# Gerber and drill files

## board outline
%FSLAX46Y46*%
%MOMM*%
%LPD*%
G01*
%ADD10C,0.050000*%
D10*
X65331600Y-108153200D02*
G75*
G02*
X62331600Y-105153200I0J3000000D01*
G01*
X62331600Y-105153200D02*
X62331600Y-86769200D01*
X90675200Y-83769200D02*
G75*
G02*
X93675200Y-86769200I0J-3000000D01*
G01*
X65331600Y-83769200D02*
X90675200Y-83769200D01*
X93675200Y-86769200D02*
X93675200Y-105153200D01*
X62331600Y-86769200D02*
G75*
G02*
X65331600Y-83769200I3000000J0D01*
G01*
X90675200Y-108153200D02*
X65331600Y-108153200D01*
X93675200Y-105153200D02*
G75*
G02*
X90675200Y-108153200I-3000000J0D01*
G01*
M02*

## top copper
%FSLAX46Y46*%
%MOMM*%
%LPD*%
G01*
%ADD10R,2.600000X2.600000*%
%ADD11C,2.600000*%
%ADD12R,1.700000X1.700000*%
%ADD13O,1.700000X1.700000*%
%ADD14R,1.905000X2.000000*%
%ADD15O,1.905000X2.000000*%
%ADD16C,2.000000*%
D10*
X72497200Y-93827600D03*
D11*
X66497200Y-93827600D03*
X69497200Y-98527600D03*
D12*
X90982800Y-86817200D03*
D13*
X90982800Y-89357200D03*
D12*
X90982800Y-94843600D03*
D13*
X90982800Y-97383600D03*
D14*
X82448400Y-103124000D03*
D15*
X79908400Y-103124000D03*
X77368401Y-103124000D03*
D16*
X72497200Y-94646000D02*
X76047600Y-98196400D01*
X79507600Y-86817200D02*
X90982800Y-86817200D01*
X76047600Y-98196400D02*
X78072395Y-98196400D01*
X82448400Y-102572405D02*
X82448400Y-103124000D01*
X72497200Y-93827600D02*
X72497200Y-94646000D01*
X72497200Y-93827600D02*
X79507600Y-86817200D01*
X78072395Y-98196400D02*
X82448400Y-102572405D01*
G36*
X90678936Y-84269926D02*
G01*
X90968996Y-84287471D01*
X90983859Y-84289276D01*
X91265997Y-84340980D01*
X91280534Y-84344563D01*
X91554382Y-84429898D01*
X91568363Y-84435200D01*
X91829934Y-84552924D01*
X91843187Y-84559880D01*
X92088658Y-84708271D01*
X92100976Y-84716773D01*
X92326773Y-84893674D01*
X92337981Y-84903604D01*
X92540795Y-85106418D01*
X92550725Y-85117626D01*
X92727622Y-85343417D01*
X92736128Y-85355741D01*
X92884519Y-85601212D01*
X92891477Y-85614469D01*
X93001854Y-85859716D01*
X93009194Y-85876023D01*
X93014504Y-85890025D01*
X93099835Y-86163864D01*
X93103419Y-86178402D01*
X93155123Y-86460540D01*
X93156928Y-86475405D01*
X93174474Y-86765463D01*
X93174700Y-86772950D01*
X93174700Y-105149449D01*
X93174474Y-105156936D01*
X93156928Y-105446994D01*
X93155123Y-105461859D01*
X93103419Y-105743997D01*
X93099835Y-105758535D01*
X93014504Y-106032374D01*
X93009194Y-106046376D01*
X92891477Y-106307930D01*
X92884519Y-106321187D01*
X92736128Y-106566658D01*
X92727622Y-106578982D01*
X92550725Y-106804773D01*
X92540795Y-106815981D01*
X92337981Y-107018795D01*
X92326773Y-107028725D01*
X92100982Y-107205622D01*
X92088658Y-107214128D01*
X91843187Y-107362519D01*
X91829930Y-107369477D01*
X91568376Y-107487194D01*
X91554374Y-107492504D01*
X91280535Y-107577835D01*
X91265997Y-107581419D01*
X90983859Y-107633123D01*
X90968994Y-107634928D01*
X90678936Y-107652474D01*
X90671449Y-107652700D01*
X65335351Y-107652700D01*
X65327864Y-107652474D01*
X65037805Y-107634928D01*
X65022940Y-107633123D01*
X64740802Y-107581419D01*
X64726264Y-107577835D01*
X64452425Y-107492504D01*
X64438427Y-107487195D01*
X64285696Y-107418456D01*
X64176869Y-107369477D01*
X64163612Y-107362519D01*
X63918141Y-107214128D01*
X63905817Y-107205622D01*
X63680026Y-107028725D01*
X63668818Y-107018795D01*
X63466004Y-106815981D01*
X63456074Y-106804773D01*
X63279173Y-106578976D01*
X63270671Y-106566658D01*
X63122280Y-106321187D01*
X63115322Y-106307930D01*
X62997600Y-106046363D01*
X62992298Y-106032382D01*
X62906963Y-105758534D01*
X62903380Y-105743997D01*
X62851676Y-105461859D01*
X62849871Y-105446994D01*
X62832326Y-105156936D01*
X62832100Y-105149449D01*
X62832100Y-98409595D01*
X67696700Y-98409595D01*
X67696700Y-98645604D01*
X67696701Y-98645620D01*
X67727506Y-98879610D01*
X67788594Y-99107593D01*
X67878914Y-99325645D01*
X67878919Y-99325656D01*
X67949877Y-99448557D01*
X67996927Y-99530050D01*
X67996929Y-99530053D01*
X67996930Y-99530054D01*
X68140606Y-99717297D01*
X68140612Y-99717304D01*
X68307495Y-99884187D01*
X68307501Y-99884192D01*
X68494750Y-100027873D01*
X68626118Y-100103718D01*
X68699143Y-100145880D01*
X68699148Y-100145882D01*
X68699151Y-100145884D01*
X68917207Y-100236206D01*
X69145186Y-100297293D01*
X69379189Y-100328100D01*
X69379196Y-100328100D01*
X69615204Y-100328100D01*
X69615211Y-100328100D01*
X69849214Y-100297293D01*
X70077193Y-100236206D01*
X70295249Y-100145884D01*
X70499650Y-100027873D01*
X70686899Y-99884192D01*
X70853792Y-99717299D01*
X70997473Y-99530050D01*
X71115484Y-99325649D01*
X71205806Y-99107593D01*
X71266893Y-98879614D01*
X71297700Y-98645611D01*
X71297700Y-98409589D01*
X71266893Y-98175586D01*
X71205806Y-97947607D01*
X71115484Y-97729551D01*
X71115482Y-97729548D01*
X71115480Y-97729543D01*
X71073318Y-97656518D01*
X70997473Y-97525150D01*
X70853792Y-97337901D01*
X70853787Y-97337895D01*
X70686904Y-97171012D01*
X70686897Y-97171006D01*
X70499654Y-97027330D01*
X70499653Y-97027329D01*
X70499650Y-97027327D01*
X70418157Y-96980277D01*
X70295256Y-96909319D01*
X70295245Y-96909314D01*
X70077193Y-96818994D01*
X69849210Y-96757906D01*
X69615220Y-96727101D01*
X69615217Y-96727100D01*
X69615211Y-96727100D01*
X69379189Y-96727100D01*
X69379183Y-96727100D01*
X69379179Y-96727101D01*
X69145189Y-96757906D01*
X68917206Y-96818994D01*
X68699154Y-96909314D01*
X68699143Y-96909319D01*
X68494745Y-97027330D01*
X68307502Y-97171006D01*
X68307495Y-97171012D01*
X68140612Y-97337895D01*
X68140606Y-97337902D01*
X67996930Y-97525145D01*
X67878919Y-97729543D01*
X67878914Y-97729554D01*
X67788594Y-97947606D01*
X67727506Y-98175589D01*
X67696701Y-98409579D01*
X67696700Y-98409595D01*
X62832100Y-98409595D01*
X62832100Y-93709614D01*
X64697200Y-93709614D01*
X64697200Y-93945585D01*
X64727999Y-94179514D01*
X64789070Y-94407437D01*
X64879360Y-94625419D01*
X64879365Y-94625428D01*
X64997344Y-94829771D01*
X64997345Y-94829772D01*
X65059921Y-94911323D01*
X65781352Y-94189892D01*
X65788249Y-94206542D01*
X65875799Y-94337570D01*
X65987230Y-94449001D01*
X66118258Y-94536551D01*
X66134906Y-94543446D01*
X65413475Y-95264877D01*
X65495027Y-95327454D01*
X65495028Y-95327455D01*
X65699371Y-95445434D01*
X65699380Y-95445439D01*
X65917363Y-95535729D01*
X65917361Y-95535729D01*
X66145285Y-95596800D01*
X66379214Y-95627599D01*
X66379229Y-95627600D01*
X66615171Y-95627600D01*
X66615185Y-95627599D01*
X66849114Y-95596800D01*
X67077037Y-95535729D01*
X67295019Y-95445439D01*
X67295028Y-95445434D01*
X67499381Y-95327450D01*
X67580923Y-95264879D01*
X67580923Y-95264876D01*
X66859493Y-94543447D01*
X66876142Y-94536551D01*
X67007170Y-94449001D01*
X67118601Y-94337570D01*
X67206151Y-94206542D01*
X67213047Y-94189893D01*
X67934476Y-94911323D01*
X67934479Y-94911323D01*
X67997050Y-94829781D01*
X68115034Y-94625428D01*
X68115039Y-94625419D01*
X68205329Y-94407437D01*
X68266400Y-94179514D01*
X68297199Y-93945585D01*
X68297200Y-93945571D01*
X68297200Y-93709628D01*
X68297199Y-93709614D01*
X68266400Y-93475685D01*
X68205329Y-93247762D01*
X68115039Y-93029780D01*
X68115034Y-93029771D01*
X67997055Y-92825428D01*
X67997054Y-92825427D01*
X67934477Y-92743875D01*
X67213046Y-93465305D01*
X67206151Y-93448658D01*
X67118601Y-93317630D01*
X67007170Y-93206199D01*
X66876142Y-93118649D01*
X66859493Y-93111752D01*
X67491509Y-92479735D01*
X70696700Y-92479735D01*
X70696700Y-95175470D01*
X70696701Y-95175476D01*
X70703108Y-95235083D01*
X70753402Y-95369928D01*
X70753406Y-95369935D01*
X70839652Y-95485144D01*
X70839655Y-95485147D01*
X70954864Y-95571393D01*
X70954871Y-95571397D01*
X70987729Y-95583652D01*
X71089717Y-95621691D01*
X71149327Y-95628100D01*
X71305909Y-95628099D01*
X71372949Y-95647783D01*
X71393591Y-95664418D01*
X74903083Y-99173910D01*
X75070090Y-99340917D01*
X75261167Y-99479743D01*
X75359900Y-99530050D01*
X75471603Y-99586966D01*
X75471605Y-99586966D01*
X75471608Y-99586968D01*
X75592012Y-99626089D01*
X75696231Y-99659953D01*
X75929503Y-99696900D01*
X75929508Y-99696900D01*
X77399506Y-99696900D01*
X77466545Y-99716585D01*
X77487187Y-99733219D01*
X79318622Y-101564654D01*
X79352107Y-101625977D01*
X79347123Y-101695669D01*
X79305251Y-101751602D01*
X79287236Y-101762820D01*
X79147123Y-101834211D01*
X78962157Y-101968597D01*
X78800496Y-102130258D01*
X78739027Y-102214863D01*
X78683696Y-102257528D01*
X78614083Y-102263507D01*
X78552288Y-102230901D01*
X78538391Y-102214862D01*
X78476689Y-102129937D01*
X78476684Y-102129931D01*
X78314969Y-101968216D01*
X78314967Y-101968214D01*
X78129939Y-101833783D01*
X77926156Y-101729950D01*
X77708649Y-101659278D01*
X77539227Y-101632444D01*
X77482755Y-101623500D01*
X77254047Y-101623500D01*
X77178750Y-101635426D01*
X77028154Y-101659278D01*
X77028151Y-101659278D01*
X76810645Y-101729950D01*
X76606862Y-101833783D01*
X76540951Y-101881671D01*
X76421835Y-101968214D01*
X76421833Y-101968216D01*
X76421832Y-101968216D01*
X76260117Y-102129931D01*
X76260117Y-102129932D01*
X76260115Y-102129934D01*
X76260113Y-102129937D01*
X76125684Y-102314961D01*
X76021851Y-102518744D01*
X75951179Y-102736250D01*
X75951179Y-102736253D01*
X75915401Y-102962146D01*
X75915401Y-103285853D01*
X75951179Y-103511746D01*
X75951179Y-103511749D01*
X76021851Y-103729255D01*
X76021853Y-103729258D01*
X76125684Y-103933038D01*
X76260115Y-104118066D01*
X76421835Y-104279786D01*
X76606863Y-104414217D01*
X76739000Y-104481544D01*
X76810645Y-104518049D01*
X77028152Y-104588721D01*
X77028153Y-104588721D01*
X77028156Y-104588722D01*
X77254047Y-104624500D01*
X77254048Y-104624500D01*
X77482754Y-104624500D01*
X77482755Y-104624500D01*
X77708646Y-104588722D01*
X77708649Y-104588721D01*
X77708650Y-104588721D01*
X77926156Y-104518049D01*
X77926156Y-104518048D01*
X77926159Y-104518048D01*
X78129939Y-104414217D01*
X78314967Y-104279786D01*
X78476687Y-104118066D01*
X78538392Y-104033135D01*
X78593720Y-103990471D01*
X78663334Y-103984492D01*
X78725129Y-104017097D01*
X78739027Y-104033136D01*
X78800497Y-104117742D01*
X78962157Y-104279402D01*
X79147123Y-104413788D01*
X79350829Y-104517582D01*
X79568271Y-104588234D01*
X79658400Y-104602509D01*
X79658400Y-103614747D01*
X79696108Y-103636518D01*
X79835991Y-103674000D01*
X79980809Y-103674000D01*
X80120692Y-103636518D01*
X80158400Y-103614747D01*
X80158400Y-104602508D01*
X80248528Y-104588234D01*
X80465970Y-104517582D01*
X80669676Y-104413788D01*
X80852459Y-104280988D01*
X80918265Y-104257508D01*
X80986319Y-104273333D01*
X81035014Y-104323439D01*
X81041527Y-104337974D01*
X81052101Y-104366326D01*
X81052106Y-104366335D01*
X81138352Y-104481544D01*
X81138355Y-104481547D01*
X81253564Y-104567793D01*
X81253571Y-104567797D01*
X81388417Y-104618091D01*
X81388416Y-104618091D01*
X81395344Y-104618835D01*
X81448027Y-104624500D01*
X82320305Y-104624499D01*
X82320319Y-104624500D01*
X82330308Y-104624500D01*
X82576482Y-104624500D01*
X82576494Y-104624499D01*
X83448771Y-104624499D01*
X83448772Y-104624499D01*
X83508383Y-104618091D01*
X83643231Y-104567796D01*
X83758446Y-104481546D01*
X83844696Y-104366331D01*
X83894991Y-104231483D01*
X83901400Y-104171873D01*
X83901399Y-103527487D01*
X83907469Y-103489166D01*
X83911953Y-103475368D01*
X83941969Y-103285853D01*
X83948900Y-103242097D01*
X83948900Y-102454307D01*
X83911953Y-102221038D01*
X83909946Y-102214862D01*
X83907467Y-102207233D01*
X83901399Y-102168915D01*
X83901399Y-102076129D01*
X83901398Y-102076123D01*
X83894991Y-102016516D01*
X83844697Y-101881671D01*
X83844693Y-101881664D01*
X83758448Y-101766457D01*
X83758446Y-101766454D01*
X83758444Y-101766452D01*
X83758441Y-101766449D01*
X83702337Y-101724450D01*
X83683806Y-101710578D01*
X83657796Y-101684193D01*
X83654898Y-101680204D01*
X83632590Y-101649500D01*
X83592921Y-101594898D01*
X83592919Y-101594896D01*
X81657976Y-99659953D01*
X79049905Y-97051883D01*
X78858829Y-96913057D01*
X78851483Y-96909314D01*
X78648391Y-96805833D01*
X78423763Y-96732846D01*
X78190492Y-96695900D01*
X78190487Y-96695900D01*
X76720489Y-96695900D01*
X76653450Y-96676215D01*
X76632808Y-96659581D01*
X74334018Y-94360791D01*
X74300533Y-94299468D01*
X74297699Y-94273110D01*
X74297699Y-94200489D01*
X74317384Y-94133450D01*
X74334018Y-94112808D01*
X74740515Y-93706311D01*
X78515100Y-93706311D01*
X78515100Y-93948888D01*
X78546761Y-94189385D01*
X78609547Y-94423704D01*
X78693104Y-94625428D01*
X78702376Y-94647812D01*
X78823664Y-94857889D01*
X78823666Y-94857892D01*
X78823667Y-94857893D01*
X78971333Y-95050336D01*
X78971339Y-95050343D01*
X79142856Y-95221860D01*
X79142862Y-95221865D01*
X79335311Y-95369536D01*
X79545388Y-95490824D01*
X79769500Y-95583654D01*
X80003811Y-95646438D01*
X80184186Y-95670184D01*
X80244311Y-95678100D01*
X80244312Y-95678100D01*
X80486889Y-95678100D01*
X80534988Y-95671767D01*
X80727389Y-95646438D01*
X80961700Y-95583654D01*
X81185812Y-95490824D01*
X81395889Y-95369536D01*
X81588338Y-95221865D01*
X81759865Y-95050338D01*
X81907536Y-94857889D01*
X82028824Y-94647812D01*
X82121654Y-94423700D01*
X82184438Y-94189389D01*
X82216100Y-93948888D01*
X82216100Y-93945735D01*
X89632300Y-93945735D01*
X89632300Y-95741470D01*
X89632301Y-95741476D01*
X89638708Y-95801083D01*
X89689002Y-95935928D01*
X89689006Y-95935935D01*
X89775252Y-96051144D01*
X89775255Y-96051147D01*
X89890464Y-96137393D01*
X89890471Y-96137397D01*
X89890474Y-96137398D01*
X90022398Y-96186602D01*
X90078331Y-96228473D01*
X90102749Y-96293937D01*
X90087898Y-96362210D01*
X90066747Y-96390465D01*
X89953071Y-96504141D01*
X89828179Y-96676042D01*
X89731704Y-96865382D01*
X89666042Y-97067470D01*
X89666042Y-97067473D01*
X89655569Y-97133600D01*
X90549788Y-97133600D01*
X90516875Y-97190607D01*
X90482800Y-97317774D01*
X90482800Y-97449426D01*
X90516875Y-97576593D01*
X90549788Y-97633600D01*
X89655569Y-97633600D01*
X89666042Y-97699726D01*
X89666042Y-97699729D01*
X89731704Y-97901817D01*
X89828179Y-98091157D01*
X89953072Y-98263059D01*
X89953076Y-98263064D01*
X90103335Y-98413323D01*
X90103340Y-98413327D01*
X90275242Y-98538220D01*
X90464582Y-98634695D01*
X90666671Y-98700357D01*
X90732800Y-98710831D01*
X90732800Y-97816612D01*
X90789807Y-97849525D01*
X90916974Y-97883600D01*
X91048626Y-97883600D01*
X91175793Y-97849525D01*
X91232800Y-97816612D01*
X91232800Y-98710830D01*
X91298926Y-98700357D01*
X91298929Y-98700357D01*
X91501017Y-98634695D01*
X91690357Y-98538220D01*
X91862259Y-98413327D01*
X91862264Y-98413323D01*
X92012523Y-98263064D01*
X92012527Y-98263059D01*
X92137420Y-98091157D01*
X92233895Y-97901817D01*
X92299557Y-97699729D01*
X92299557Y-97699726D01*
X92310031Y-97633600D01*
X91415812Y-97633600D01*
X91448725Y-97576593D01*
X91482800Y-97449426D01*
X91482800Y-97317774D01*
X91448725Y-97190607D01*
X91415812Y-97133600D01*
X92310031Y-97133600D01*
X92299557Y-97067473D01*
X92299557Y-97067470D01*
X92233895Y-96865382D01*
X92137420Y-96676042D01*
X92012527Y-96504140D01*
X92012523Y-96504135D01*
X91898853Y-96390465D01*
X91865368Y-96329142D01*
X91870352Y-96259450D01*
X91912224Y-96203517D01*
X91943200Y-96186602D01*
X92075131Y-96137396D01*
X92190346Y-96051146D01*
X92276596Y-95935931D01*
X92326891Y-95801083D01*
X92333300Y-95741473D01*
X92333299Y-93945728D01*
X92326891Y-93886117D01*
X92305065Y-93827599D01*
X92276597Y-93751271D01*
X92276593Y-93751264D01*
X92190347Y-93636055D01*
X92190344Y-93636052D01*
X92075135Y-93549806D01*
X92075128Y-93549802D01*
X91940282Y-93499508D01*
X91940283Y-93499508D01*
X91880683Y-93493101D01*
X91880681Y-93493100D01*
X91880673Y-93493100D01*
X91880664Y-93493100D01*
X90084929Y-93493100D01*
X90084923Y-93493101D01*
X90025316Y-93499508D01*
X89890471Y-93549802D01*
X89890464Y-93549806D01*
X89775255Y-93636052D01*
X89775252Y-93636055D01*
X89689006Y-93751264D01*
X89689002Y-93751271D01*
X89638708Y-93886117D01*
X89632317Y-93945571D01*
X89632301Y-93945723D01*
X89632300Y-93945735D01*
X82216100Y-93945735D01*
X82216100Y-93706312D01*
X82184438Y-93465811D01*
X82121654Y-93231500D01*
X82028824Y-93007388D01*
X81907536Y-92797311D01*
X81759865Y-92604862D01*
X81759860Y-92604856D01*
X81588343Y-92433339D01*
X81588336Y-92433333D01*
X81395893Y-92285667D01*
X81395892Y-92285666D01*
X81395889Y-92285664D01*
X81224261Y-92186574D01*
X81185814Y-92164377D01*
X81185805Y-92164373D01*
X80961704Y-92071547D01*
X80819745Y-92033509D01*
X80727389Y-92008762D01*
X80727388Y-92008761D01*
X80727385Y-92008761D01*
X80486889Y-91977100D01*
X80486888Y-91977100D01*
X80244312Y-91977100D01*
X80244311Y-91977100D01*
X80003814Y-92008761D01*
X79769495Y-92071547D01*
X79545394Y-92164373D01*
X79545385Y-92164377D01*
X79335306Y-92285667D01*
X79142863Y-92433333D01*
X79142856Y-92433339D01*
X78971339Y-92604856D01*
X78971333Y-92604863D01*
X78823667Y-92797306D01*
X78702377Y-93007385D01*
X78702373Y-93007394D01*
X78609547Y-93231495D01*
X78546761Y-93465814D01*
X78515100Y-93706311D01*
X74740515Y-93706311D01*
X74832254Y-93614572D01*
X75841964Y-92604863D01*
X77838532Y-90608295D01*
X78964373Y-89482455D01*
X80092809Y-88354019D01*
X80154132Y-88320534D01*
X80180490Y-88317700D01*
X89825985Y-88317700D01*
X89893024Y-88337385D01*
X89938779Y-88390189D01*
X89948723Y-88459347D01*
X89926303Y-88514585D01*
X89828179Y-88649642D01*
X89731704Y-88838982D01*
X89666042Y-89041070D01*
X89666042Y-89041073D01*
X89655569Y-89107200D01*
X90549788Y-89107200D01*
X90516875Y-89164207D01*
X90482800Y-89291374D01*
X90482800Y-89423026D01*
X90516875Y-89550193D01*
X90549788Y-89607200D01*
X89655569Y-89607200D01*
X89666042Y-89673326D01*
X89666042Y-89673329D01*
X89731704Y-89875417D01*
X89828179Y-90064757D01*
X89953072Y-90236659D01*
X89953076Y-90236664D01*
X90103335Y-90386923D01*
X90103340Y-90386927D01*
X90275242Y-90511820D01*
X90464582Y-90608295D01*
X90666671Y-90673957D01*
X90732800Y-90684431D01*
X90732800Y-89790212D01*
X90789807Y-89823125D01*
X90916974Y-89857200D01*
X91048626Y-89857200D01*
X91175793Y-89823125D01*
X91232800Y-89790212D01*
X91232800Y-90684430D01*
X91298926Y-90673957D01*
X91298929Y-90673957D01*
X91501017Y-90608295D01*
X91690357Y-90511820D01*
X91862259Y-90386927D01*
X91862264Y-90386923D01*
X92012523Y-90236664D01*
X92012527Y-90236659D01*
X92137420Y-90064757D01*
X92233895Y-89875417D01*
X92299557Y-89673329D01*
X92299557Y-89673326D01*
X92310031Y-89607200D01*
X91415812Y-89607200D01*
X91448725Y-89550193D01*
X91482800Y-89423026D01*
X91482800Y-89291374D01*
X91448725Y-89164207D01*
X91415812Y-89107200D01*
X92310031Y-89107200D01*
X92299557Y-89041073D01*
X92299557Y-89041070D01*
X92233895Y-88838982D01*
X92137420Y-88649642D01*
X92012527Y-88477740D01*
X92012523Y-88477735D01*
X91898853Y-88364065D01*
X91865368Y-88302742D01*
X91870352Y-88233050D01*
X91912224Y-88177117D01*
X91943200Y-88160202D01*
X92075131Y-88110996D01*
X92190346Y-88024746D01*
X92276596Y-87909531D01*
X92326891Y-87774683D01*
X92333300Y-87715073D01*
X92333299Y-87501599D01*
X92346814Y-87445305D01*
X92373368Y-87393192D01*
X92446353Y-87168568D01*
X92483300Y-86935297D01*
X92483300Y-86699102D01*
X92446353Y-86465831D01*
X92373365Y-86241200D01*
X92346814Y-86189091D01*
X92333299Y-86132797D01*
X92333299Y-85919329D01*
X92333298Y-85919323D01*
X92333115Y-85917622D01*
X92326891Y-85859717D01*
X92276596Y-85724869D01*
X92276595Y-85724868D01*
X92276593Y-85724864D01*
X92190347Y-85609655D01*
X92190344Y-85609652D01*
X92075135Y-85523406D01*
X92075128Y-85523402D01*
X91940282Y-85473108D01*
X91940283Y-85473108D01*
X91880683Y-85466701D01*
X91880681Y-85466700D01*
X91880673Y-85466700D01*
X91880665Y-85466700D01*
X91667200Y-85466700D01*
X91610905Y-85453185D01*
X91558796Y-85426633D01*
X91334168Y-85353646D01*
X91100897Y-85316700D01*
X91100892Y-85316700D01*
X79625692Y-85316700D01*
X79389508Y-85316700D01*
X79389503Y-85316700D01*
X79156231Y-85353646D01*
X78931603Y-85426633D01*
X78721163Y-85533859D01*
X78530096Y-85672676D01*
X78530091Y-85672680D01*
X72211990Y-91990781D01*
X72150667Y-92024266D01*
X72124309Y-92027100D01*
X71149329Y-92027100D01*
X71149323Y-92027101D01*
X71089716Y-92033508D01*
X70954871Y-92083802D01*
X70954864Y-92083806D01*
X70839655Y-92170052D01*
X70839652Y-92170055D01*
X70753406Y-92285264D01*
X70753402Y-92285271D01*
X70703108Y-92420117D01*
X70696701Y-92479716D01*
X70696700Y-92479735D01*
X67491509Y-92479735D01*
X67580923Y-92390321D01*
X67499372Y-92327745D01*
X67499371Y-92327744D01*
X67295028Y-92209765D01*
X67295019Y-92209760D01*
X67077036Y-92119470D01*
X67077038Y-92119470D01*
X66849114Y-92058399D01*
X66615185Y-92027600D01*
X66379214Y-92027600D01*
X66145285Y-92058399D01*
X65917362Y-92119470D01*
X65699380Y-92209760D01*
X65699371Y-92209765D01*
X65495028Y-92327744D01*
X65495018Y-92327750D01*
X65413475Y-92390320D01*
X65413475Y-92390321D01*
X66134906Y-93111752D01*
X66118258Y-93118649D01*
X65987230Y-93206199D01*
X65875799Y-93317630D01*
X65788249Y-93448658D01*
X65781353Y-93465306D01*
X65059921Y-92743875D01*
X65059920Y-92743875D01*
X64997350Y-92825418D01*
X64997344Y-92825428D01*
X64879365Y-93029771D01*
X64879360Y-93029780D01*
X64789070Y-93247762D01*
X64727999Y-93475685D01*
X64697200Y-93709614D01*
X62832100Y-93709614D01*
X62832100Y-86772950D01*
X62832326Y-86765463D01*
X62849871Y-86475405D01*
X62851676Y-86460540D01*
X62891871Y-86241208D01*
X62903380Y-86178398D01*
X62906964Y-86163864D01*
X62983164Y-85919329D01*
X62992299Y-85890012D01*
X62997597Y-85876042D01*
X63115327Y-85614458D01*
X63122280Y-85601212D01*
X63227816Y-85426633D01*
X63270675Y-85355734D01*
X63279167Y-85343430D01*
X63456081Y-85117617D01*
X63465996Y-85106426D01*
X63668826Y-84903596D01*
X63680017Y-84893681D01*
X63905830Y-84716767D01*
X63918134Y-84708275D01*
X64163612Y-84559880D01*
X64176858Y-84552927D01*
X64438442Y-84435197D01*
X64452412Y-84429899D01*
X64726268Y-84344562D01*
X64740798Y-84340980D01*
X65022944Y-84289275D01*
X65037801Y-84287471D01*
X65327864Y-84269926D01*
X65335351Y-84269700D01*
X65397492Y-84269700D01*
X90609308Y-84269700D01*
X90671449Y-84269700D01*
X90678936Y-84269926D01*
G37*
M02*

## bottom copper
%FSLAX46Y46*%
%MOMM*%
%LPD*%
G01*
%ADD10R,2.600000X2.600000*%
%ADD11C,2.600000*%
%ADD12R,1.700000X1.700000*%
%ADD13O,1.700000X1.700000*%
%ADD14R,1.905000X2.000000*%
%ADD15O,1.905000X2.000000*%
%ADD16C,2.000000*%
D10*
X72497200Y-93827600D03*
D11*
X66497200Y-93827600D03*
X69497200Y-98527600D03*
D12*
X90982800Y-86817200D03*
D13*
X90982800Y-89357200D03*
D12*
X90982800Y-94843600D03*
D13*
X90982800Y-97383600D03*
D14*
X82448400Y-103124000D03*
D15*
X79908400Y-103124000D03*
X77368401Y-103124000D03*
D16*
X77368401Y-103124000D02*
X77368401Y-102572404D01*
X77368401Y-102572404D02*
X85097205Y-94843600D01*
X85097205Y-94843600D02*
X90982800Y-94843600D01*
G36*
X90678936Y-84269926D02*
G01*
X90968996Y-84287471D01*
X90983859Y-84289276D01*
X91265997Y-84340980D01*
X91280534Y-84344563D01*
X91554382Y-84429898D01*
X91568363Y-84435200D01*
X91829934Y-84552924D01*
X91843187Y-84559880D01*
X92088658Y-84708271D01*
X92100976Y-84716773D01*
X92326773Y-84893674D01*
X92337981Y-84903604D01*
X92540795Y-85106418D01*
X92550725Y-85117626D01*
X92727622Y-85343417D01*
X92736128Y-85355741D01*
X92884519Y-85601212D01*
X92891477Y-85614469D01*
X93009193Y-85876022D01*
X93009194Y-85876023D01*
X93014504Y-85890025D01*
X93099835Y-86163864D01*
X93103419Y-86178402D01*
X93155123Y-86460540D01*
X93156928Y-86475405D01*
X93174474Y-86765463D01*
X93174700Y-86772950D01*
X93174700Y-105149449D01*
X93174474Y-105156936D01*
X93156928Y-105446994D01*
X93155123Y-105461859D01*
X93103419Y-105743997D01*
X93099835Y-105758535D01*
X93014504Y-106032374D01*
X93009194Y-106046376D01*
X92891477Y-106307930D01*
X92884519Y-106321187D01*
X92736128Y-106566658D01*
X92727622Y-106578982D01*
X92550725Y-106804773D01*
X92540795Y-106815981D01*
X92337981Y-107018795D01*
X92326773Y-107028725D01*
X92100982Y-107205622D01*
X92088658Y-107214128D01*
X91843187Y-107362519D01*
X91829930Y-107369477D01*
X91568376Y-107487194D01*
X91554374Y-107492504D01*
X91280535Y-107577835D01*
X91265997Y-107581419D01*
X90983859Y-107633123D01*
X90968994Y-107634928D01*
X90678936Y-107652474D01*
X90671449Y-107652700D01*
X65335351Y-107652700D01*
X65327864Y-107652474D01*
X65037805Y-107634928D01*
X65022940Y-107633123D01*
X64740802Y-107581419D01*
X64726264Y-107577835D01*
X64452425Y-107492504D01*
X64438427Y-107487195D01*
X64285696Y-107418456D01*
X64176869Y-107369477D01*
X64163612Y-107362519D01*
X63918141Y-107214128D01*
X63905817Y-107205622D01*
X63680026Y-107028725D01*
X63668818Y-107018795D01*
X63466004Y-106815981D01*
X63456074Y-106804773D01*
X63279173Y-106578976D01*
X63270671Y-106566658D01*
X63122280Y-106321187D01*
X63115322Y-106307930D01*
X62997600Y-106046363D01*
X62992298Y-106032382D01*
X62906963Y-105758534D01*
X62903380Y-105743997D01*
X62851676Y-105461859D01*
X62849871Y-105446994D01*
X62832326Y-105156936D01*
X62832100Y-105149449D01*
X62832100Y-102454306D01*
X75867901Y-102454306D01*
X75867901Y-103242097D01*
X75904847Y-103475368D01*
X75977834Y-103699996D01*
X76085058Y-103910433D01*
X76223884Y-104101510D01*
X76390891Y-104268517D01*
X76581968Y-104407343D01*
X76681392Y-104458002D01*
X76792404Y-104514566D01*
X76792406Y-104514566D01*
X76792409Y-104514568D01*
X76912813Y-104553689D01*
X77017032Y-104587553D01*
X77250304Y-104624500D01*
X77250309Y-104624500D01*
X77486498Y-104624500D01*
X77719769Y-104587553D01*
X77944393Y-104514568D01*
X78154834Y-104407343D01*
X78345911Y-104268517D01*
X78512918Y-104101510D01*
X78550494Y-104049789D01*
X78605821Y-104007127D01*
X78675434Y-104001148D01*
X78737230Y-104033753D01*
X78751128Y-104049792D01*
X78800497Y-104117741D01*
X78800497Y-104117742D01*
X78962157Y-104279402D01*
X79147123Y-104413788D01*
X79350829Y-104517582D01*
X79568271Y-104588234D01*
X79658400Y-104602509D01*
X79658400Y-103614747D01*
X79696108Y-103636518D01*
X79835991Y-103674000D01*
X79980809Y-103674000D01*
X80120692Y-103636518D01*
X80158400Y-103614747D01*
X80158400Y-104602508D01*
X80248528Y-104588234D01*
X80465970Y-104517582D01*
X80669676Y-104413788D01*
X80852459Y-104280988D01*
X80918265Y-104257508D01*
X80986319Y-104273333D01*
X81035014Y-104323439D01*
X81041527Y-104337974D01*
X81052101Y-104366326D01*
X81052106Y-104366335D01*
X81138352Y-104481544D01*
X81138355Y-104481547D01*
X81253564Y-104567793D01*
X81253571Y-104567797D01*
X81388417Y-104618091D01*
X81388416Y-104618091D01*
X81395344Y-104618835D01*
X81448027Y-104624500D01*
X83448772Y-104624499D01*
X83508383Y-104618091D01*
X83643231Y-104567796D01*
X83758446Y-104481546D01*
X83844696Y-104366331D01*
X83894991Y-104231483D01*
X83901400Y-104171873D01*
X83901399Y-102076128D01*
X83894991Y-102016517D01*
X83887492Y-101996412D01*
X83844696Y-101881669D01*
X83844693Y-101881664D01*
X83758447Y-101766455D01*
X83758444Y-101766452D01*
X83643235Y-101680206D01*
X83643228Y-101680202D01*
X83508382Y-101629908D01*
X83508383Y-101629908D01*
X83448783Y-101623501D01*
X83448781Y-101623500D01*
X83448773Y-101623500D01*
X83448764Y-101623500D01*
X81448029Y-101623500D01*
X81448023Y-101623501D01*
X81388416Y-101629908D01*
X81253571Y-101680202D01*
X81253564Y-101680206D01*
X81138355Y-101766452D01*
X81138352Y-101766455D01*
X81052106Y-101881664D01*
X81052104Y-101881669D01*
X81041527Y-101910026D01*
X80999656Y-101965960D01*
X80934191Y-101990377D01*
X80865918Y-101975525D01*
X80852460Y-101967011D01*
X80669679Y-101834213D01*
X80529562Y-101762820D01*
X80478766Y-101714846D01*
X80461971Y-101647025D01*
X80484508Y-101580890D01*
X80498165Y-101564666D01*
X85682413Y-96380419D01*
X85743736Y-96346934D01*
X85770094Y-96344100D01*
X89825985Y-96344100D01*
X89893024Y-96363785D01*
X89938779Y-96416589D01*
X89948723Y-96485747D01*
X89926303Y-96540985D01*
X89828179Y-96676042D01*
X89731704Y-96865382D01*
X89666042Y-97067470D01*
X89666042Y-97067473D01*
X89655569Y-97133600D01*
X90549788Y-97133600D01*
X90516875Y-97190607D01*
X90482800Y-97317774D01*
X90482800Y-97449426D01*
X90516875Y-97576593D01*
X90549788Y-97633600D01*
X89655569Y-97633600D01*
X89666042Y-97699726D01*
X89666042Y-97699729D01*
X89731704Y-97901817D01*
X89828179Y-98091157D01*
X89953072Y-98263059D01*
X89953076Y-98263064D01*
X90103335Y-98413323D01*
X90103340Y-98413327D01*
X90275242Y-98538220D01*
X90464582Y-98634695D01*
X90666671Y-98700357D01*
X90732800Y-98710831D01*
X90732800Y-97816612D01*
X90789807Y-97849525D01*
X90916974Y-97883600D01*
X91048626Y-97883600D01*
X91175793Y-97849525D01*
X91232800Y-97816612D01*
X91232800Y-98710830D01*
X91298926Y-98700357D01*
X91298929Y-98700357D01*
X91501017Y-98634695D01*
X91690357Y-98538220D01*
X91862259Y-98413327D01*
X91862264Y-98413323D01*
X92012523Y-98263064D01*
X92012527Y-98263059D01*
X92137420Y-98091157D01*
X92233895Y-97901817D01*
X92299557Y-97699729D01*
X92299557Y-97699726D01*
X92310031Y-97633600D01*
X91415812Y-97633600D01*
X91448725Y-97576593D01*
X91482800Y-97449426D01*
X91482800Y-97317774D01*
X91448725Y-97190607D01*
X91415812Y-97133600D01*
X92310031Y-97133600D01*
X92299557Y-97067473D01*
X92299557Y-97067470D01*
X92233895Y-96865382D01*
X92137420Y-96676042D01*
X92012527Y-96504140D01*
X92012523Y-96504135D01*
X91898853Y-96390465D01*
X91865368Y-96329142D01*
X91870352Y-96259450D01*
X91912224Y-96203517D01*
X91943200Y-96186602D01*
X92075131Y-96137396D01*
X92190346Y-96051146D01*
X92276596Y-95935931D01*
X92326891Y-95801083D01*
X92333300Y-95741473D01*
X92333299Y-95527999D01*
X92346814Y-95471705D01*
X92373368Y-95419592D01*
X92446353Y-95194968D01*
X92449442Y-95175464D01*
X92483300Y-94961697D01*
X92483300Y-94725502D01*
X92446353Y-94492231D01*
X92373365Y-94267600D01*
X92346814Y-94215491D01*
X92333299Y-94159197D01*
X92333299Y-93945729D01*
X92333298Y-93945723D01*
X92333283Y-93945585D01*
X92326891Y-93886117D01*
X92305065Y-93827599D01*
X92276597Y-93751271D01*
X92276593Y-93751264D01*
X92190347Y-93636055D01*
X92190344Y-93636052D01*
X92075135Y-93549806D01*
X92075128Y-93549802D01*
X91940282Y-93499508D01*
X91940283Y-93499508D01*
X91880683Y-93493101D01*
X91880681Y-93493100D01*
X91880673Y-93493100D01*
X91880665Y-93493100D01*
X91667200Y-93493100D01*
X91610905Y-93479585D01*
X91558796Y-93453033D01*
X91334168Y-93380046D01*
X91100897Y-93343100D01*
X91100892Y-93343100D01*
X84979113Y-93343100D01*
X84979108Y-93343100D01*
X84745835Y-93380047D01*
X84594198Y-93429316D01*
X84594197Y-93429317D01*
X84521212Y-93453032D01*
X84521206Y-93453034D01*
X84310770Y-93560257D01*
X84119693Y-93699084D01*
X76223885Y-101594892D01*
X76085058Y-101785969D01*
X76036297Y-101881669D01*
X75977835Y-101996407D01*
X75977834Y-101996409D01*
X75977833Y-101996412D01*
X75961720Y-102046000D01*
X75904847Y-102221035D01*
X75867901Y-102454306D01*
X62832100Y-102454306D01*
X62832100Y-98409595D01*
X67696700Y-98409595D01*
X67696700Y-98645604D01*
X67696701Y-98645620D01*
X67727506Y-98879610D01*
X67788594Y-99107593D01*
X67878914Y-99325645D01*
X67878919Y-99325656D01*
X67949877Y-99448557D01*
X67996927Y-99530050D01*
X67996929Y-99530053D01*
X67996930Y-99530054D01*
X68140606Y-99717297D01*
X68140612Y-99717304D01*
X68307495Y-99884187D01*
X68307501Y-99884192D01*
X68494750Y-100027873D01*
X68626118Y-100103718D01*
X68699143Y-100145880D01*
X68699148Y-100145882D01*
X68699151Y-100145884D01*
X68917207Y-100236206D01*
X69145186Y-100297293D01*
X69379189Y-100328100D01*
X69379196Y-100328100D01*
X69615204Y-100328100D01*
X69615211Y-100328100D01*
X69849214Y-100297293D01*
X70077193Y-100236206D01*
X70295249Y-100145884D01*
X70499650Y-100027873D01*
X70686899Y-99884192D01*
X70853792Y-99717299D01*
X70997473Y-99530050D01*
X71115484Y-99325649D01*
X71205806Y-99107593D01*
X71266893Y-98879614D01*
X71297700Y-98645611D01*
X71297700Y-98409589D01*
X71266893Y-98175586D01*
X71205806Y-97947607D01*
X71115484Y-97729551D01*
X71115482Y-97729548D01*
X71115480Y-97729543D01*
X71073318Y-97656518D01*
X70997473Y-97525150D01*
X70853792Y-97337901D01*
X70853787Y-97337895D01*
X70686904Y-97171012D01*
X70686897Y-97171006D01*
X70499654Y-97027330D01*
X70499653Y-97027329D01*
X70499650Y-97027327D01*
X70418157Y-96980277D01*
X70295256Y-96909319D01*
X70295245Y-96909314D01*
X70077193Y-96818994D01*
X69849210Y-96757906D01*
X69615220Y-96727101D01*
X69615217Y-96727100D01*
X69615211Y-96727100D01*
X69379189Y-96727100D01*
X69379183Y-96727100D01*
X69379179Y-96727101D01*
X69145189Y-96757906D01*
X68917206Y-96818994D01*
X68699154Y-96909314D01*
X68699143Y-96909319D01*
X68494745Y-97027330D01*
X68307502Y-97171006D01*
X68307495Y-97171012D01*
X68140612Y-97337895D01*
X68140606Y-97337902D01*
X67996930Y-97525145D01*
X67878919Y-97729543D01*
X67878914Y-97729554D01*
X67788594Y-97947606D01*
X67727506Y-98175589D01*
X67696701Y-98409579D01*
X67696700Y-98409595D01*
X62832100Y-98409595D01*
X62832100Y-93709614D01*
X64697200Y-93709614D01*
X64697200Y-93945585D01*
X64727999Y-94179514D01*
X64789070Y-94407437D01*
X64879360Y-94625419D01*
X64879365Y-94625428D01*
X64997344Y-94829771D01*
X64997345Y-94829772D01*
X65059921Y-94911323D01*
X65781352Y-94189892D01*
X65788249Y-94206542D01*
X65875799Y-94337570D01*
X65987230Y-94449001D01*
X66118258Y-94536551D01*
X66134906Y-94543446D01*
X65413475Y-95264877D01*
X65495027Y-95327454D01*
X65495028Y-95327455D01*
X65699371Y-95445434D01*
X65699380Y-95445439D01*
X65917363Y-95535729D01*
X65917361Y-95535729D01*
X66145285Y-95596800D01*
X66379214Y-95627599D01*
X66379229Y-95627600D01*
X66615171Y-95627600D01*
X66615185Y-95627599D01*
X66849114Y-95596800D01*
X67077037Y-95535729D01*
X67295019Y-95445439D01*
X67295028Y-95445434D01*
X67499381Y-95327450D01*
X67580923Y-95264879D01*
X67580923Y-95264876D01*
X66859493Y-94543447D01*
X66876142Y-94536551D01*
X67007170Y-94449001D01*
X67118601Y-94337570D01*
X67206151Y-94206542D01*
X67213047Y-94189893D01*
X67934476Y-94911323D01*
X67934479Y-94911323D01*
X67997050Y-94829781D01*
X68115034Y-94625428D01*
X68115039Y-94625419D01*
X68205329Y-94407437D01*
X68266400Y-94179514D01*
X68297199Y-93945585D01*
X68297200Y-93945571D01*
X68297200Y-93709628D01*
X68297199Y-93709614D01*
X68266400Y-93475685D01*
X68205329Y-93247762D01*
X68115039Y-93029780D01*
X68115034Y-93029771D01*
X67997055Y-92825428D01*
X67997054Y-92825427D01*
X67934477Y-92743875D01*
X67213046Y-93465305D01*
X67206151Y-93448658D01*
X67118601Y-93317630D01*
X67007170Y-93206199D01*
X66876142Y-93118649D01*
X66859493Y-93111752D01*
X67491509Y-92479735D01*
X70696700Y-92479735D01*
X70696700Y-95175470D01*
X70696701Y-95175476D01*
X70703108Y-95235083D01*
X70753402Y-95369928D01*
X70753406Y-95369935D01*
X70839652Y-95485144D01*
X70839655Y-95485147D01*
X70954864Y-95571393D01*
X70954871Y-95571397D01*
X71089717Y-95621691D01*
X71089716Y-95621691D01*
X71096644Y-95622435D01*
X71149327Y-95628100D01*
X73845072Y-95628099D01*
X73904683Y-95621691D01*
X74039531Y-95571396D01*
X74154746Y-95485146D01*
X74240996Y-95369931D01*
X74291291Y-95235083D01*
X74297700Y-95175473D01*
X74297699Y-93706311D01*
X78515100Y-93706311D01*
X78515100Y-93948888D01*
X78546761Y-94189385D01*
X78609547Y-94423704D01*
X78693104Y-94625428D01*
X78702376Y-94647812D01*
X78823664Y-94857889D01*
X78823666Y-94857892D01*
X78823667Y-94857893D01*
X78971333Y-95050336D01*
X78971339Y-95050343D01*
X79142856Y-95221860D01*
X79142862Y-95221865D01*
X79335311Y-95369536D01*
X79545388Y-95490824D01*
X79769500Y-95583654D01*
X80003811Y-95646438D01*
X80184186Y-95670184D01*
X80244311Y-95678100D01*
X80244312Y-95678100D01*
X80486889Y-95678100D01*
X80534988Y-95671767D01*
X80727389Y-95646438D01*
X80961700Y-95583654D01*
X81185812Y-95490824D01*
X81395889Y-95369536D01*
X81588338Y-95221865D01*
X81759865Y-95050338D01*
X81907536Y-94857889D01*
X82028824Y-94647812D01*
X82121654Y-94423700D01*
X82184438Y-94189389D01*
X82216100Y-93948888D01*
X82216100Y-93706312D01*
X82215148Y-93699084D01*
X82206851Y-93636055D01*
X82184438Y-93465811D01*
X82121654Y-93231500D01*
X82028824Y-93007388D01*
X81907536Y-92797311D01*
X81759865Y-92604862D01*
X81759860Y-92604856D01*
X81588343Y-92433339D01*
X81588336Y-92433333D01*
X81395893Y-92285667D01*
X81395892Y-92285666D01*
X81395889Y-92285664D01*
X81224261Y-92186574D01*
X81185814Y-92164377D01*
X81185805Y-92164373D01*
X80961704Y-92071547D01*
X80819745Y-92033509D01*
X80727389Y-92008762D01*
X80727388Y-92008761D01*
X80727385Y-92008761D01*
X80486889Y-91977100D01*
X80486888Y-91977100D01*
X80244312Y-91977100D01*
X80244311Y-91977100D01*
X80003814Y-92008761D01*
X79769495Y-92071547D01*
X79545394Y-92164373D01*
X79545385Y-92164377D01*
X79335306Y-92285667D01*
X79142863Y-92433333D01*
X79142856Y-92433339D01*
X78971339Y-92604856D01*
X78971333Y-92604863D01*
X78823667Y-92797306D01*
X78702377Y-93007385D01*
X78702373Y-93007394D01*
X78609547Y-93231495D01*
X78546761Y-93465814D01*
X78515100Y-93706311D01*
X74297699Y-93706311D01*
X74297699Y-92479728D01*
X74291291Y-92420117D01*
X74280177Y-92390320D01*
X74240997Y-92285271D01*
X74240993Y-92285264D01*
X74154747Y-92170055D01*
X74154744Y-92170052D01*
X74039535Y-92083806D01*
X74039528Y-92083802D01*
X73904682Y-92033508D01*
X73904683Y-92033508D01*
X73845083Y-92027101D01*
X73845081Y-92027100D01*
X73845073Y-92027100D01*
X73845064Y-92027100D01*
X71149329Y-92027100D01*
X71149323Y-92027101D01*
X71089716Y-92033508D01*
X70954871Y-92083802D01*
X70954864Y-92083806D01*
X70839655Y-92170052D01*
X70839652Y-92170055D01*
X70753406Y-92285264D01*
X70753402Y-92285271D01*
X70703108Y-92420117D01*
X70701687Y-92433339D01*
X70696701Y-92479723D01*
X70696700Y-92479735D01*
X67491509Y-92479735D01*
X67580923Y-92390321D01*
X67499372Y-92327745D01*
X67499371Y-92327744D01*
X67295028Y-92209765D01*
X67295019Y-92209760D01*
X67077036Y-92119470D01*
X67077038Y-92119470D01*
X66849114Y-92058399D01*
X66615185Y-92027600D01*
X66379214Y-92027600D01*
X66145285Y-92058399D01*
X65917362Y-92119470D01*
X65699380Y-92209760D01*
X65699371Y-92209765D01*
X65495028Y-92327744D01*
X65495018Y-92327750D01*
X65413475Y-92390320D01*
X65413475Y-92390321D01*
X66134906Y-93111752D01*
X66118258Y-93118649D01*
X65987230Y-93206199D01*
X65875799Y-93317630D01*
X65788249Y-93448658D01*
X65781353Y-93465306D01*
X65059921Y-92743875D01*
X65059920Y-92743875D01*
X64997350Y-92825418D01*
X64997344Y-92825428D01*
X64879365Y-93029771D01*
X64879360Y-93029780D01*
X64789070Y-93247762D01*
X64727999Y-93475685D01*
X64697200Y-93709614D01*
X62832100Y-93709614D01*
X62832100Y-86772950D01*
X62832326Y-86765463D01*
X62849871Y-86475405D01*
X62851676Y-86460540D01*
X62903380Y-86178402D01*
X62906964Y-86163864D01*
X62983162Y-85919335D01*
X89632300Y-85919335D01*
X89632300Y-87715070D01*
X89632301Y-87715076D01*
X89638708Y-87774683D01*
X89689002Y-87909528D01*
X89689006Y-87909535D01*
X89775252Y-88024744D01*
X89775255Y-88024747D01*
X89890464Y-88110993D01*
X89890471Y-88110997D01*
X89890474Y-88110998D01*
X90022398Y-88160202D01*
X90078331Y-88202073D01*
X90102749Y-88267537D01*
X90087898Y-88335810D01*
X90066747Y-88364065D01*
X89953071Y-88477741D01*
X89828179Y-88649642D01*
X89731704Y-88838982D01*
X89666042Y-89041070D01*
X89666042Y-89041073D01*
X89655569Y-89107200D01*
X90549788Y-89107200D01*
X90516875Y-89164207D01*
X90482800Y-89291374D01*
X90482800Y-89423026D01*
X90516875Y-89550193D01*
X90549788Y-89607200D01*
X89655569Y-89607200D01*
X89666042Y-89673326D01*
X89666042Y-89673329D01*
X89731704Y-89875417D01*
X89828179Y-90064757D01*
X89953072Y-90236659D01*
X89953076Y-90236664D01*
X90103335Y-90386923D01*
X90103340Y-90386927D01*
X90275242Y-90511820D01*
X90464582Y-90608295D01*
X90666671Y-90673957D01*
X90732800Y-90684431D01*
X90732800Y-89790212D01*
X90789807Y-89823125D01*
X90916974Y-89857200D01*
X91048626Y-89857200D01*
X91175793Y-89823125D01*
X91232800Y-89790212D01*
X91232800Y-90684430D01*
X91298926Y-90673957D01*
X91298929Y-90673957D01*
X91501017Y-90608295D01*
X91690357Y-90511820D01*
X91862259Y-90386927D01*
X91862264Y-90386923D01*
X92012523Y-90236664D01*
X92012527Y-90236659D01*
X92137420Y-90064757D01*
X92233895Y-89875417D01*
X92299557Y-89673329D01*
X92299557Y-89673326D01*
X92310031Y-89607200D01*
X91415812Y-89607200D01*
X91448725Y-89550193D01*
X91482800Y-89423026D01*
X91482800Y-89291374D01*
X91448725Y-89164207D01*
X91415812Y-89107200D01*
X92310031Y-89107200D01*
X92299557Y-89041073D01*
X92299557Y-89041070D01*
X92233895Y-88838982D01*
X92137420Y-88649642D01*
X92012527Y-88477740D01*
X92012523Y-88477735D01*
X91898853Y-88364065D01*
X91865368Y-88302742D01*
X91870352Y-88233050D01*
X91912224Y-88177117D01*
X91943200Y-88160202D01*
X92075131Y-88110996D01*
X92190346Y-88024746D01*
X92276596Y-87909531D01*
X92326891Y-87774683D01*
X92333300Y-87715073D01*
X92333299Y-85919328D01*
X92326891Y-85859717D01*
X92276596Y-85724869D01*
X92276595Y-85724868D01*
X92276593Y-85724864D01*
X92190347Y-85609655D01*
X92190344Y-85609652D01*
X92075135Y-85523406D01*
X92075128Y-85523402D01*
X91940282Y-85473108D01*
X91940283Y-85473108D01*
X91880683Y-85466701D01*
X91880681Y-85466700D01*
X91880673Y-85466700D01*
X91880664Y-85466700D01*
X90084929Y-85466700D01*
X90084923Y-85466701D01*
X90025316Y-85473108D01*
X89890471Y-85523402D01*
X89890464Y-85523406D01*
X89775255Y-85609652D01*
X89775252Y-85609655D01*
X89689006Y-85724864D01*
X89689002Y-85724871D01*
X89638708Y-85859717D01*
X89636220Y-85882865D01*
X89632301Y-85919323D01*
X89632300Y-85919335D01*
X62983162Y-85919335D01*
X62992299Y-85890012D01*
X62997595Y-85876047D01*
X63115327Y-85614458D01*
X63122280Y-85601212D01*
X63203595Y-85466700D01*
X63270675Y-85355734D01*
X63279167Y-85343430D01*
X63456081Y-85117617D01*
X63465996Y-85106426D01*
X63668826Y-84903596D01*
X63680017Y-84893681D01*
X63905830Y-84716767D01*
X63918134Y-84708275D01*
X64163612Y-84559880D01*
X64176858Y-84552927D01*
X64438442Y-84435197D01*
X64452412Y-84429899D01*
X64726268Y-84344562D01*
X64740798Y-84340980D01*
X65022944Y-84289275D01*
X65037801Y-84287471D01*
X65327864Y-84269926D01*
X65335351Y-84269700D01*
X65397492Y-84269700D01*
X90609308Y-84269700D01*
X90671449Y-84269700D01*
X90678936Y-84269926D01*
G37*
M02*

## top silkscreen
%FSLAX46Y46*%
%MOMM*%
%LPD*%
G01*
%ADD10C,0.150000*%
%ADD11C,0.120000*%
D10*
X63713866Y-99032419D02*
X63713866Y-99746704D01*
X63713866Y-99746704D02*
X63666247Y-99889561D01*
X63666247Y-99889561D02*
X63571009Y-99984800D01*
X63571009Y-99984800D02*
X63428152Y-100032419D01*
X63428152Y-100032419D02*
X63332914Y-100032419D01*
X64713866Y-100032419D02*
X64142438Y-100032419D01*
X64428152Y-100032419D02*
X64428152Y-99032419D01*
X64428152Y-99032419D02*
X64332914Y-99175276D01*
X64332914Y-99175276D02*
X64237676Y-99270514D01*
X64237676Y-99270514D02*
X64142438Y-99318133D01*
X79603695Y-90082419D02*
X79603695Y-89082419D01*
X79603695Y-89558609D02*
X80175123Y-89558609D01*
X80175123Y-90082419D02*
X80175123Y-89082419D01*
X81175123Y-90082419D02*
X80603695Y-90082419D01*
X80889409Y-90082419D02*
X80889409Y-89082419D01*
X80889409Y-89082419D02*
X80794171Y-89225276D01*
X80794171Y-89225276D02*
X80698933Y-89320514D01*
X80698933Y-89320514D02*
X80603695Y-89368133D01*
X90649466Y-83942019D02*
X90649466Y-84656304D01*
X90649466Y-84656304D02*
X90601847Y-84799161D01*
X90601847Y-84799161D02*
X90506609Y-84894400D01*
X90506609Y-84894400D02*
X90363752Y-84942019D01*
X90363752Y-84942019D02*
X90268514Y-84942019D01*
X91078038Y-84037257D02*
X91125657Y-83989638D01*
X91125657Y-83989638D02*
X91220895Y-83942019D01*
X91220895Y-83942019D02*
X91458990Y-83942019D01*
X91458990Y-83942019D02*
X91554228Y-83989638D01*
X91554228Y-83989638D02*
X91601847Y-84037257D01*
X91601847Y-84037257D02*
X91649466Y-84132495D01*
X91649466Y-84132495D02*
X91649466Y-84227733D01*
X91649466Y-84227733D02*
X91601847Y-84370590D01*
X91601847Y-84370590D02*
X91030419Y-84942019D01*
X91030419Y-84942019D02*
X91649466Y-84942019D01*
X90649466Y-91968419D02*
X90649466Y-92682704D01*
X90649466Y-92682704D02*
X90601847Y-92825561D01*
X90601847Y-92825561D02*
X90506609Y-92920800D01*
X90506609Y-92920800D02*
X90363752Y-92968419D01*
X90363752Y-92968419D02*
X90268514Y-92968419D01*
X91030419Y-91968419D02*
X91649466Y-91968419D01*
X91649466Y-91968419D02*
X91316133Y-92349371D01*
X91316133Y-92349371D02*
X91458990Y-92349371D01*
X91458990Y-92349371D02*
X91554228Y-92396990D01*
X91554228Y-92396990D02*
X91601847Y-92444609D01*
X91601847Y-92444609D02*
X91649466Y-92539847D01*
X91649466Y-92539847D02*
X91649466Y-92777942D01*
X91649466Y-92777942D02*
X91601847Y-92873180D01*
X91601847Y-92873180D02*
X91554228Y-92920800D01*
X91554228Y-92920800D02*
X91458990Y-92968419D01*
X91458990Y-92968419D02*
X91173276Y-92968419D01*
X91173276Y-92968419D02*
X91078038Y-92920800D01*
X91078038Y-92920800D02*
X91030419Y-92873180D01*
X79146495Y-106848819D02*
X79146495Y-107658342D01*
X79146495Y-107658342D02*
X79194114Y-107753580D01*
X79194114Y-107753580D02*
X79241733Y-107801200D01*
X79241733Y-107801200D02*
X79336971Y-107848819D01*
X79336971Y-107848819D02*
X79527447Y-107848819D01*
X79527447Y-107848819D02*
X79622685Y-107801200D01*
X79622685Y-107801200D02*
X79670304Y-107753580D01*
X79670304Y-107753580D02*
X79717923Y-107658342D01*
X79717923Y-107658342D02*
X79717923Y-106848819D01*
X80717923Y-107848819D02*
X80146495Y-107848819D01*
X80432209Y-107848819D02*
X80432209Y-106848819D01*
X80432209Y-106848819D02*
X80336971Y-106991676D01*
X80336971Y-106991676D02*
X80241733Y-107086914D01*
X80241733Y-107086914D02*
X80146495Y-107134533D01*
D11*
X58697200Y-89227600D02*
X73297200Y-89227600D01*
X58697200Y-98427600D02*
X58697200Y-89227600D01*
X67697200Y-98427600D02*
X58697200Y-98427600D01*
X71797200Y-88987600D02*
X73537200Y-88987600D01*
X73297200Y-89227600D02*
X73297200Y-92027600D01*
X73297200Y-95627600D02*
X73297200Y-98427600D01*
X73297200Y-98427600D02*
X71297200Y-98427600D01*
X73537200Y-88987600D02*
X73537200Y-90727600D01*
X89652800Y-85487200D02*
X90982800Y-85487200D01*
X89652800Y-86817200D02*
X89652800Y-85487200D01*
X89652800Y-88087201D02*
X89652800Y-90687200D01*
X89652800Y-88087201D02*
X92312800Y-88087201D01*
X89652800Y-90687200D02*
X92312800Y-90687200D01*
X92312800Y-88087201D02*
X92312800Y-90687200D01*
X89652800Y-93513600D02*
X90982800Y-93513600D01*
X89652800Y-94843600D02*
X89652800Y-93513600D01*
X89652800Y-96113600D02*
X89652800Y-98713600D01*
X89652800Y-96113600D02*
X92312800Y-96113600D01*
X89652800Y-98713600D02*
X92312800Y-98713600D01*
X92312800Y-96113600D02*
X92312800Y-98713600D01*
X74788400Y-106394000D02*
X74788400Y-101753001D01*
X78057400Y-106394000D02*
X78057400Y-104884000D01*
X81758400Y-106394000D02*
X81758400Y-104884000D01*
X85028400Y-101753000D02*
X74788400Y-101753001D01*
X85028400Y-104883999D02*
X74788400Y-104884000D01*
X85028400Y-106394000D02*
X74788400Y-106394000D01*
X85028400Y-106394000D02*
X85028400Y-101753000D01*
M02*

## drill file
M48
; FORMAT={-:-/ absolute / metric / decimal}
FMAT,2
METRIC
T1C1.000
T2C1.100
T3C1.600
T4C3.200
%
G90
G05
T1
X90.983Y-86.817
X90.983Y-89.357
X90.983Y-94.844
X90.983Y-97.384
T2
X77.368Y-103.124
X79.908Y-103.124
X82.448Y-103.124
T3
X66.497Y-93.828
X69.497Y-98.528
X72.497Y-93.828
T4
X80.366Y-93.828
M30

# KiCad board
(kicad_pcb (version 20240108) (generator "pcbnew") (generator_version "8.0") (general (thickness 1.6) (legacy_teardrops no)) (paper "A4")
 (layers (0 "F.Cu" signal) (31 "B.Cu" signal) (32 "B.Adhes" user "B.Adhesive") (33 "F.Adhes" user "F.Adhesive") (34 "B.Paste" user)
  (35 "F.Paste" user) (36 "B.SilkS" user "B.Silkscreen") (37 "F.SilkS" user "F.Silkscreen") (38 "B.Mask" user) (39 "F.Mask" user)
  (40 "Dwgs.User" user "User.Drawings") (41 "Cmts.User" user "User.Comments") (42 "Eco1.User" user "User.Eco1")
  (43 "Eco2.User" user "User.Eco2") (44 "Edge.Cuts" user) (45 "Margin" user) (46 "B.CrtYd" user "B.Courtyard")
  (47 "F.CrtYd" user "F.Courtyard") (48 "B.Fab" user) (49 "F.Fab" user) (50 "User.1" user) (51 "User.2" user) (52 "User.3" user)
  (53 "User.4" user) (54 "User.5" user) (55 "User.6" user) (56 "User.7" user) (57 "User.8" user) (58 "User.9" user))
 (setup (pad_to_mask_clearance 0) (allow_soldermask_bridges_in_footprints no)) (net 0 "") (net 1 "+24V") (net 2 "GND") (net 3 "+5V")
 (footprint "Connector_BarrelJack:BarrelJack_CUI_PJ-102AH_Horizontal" (layer "F.Cu") (at 72.4972 93.8276 -90)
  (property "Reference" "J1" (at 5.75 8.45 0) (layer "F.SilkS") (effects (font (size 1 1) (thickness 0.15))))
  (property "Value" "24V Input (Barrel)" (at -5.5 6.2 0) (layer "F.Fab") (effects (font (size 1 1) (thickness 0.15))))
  (fp_line (start -4.6 13.8) (end -4.6 -0.8) (stroke (width 0.12) (type solid)) (layer "F.SilkS"))
  (fp_line (start 4.6 13.8) (end -4.6 13.8) (stroke (width 0.12) (type solid)) (layer "F.SilkS"))
  (fp_line (start 4.6 4.8) (end 4.6 13.8) (stroke (width 0.12) (type solid)) (layer "F.SilkS"))
  (fp_line (start -4.84 0.7) (end -4.84 -1.04) (stroke (width 0.12) (type solid)) (layer "F.SilkS"))
  (fp_line (start -4.6 -0.8) (end -1.8 -0.8) (stroke (width 0.12) (type solid)) (layer "F.SilkS"))
  (fp_line (start 1.8 -0.8) (end 4.6 -0.8) (stroke (width 0.12) (type solid)) (layer "F.SilkS"))
  (fp_line (start 4.6 -0.8) (end 4.6 1.2) (stroke (width 0.12) (type solid)) (layer "F.SilkS"))
  (fp_line (start -4.84 -1.04) (end -3.1 -1.04) (stroke (width 0.12) (type solid)) (layer "F.SilkS"))
  (pad "1" thru_hole rect (at 0 0 270) (size 2.6 2.6) (drill 1.6) (layers "*.Cu" "*.Mask") (remove_unused_layers no) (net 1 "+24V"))
  (pad "2" thru_hole circle (at 0 6 270) (size 2.6 2.6) (drill 1.6) (layers "*.Cu" "*.Mask") (remove_unused_layers no) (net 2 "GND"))
  (pad "3" thru_hole circle (at 4.7 3 270) (size 2.6 2.6) (drill 1.6) (layers "*.Cu" "*.Mask") (remove_unused_layers no)))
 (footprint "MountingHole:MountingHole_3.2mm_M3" (layer "F.Cu") (at 80.3656 93.8276)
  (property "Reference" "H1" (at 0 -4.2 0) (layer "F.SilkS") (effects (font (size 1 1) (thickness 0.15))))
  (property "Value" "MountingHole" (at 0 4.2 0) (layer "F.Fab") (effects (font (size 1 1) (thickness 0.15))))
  (pad "" np_thru_hole circle (at 0 0) (size 3.2 3.2) (drill 3.2) (layers "*.Cu" "*.Mask")))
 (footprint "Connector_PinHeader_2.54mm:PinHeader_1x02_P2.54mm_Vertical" (layer "F.Cu") (at 90.9828 86.8172)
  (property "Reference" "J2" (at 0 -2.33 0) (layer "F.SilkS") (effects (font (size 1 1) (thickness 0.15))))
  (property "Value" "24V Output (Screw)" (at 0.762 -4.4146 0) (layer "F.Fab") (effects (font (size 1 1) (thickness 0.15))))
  (fp_line (start -1.33 -1.33) (end 0 -1.33) (stroke (width 0.12) (type solid)) (layer "F.SilkS"))
  (fp_line (start -1.33 0) (end -1.33 -1.33) (stroke (width 0.12) (type solid)) (layer "F.SilkS"))
  (fp_line (start -1.33 1.270001) (end -1.33 3.87) (stroke (width 0.12) (type solid)) (layer "F.SilkS"))
  (fp_line (start -1.33 1.270001) (end 1.33 1.270001) (stroke (width 0.12) (type solid)) (layer "F.SilkS"))
  (fp_line (start -1.33 3.87) (end 1.33 3.87) (stroke (width 0.12) (type solid)) (layer "F.SilkS"))
  (fp_line (start 1.33 1.270001) (end 1.33 3.87) (stroke (width 0.12) (type solid)) (layer "F.SilkS"))
  (pad "1" thru_hole rect (at 0 0) (size 1.7 1.7) (drill 1) (layers "*.Cu" "*.Mask") (remove_unused_layers no) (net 1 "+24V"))
  (pad "2" thru_hole oval (at 0 2.54) (size 1.7 1.7) (drill 1) (layers "*.Cu" "*.Mask") (remove_unused_layers no) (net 2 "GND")))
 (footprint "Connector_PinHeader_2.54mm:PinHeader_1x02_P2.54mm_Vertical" (layer "F.Cu") (at 90.9828 94.8436)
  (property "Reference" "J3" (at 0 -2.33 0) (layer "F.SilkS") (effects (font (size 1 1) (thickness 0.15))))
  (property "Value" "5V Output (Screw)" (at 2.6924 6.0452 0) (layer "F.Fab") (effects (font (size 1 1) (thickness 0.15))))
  (fp_line (start -1.33 -1.33) (end 0 -1.33) (stroke (width 0.12) (type solid)) (layer "F.SilkS"))
  (fp_line (start -1.33 0) (end -1.33 -1.33) (stroke (width 0.12) (type solid)) (layer "F.SilkS"))
  (fp_line (start -1.33 1.27) (end -1.33 3.87) (stroke (width 0.12) (type solid)) (layer "F.SilkS"))
  (fp_line (start -1.33 1.27) (end 1.33 1.27) (stroke (width 0.12) (type solid)) (layer "F.SilkS"))
  (fp_line (start -1.33 3.87) (end 1.33 3.87) (stroke (width 0.12) (type solid)) (layer "F.SilkS"))
  (fp_line (start 1.33 1.27) (end 1.33 3.87) (stroke (width 0.12) (type solid)) (layer "F.SilkS"))
  (pad "1" thru_hole rect (at 0 0) (size 1.7 1.7) (drill 1) (layers "*.Cu" "*.Mask") (remove_unused_layers no) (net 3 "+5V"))
  (pad "2" thru_hole oval (at 0 2.54) (size 1.7 1.7) (drill 1) (layers "*.Cu" "*.Mask") (remove_unused_layers no) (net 2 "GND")))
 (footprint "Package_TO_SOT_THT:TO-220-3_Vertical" (layer "F.Cu") (at 82.4484 103.124 180)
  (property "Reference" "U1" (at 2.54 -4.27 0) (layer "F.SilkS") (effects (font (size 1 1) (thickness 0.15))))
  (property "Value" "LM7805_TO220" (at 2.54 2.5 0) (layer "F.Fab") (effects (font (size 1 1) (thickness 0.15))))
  (fp_line (start 7.66 -3.27) (end 7.66 1.370999) (stroke (width 0.12) (type solid)) (layer "F.SilkS"))
  (fp_line (start 4.391 -3.27) (end 4.391 -1.76) (stroke (width 0.12) (type solid)) (layer "F.SilkS"))
  (fp_line (start 0.69 -3.27) (end 0.69 -1.76) (stroke (width 0.12) (type solid)) (layer "F.SilkS"))
  (fp_line (start -2.58 1.371) (end 7.66 1.370999) (stroke (width 0.12) (type solid)) (layer "F.SilkS"))
  (fp_line (start -2.58 -1.759999) (end 7.66 -1.76) (stroke (width 0.12) (type solid)) (layer "F.SilkS"))
  (fp_line (start -2.58 -3.27) (end 7.66 -3.27) (stroke (width 0.12) (type solid)) (layer "F.SilkS"))
  (fp_line (start -2.58 -3.27) (end -2.58 1.371) (stroke (width 0.12) (type solid)) (layer "F.SilkS"))
  (pad "1" thru_hole rect (at 0 0 180) (size 1.905 2) (drill 1.1) (layers "*.Cu" "*.Mask") (remove_unused_layers no) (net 1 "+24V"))
  (pad "2" thru_hole oval (at 2.54 0 180) (size 1.905 2) (drill 1.1) (layers "*.Cu" "*.Mask") (remove_unused_layers no) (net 2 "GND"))
  (pad "3" thru_hole oval (at 5.079999 0 180) (size 1.905 2) (drill 1.1) (layers "*.Cu" "*.Mask") (remove_unused_layers no) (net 3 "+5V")))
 (gr_arc (start 65.3316 108.1532) (mid 63.21028 107.27452) (end 62.3316 105.1532) (stroke (width 0.05) (type default)) (layer "Edge.Cuts"))
 (gr_line (start 62.3316 105.1532) (end 62.3316 86.7692) (stroke (width 0.05) (type default)) (layer "Edge.Cuts"))
 (gr_arc (start 90.6752 83.7692) (mid 92.79652 84.64788) (end 93.6752 86.7692) (stroke (width 0.05) (type default)) (layer "Edge.Cuts"))
 (gr_line (start 65.3316 83.7692) (end 90.6752 83.7692) (stroke (width 0.05) (type default)) (layer "Edge.Cuts"))
 (gr_line (start 93.6752 86.7692) (end 93.6752 105.1532) (stroke (width 0.05) (type default)) (layer "Edge.Cuts"))
 (gr_arc (start 62.3316 86.7692) (mid 63.21028 84.64788) (end 65.3316 83.7692) (stroke (width 0.05) (type default)) (layer "Edge.Cuts"))
 (gr_line (start 90.6752 108.1532) (end 65.3316 108.1532) (stroke (width 0.05) (type default)) (layer "Edge.Cuts"))
 (gr_arc (start 93.6752 105.1532) (mid 92.79652 107.27452) (end 90.6752 108.1532) (stroke (width 0.05) (type default)) (layer "Edge.Cuts"))
 (segment (start 72.4972 94.646) (end 76.0476 98.1964) (width 2) (layer "F.Cu") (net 1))
 (segment (start 79.5076 86.8172) (end 90.9828 86.8172) (width 2) (layer "F.Cu") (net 1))
 (segment (start 76.0476 98.1964) (end 78.072395 98.1964) (width 2) (layer "F.Cu") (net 1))
 (segment (start 82.4484 102.572405) (end 82.4484 103.124) (width 2) (layer "F.Cu") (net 1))
 (segment (start 72.4972 93.8276) (end 72.4972 94.646) (width 2) (layer "F.Cu") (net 1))
 (segment (start 72.4972 93.8276) (end 79.5076 86.8172) (width 2) (layer "F.Cu") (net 1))
 (segment (start 78.072395 98.1964) (end 82.4484 102.572405) (width 2) (layer "F.Cu") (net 1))
 (segment (start 77.368401 103.124) (end 77.368401 102.572404) (width 2) (layer "B.Cu") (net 3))
 (segment (start 77.368401 102.572404) (end 85.097205 94.8436) (width 2) (layer "B.Cu") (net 3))
 (segment (start 85.097205 94.8436) (end 90.9828 94.8436) (width 2) (layer "B.Cu") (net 3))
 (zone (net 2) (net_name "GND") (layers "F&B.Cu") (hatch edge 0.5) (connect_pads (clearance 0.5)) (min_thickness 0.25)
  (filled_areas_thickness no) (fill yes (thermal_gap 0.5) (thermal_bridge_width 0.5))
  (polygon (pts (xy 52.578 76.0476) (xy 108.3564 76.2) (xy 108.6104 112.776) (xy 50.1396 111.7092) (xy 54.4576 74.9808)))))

